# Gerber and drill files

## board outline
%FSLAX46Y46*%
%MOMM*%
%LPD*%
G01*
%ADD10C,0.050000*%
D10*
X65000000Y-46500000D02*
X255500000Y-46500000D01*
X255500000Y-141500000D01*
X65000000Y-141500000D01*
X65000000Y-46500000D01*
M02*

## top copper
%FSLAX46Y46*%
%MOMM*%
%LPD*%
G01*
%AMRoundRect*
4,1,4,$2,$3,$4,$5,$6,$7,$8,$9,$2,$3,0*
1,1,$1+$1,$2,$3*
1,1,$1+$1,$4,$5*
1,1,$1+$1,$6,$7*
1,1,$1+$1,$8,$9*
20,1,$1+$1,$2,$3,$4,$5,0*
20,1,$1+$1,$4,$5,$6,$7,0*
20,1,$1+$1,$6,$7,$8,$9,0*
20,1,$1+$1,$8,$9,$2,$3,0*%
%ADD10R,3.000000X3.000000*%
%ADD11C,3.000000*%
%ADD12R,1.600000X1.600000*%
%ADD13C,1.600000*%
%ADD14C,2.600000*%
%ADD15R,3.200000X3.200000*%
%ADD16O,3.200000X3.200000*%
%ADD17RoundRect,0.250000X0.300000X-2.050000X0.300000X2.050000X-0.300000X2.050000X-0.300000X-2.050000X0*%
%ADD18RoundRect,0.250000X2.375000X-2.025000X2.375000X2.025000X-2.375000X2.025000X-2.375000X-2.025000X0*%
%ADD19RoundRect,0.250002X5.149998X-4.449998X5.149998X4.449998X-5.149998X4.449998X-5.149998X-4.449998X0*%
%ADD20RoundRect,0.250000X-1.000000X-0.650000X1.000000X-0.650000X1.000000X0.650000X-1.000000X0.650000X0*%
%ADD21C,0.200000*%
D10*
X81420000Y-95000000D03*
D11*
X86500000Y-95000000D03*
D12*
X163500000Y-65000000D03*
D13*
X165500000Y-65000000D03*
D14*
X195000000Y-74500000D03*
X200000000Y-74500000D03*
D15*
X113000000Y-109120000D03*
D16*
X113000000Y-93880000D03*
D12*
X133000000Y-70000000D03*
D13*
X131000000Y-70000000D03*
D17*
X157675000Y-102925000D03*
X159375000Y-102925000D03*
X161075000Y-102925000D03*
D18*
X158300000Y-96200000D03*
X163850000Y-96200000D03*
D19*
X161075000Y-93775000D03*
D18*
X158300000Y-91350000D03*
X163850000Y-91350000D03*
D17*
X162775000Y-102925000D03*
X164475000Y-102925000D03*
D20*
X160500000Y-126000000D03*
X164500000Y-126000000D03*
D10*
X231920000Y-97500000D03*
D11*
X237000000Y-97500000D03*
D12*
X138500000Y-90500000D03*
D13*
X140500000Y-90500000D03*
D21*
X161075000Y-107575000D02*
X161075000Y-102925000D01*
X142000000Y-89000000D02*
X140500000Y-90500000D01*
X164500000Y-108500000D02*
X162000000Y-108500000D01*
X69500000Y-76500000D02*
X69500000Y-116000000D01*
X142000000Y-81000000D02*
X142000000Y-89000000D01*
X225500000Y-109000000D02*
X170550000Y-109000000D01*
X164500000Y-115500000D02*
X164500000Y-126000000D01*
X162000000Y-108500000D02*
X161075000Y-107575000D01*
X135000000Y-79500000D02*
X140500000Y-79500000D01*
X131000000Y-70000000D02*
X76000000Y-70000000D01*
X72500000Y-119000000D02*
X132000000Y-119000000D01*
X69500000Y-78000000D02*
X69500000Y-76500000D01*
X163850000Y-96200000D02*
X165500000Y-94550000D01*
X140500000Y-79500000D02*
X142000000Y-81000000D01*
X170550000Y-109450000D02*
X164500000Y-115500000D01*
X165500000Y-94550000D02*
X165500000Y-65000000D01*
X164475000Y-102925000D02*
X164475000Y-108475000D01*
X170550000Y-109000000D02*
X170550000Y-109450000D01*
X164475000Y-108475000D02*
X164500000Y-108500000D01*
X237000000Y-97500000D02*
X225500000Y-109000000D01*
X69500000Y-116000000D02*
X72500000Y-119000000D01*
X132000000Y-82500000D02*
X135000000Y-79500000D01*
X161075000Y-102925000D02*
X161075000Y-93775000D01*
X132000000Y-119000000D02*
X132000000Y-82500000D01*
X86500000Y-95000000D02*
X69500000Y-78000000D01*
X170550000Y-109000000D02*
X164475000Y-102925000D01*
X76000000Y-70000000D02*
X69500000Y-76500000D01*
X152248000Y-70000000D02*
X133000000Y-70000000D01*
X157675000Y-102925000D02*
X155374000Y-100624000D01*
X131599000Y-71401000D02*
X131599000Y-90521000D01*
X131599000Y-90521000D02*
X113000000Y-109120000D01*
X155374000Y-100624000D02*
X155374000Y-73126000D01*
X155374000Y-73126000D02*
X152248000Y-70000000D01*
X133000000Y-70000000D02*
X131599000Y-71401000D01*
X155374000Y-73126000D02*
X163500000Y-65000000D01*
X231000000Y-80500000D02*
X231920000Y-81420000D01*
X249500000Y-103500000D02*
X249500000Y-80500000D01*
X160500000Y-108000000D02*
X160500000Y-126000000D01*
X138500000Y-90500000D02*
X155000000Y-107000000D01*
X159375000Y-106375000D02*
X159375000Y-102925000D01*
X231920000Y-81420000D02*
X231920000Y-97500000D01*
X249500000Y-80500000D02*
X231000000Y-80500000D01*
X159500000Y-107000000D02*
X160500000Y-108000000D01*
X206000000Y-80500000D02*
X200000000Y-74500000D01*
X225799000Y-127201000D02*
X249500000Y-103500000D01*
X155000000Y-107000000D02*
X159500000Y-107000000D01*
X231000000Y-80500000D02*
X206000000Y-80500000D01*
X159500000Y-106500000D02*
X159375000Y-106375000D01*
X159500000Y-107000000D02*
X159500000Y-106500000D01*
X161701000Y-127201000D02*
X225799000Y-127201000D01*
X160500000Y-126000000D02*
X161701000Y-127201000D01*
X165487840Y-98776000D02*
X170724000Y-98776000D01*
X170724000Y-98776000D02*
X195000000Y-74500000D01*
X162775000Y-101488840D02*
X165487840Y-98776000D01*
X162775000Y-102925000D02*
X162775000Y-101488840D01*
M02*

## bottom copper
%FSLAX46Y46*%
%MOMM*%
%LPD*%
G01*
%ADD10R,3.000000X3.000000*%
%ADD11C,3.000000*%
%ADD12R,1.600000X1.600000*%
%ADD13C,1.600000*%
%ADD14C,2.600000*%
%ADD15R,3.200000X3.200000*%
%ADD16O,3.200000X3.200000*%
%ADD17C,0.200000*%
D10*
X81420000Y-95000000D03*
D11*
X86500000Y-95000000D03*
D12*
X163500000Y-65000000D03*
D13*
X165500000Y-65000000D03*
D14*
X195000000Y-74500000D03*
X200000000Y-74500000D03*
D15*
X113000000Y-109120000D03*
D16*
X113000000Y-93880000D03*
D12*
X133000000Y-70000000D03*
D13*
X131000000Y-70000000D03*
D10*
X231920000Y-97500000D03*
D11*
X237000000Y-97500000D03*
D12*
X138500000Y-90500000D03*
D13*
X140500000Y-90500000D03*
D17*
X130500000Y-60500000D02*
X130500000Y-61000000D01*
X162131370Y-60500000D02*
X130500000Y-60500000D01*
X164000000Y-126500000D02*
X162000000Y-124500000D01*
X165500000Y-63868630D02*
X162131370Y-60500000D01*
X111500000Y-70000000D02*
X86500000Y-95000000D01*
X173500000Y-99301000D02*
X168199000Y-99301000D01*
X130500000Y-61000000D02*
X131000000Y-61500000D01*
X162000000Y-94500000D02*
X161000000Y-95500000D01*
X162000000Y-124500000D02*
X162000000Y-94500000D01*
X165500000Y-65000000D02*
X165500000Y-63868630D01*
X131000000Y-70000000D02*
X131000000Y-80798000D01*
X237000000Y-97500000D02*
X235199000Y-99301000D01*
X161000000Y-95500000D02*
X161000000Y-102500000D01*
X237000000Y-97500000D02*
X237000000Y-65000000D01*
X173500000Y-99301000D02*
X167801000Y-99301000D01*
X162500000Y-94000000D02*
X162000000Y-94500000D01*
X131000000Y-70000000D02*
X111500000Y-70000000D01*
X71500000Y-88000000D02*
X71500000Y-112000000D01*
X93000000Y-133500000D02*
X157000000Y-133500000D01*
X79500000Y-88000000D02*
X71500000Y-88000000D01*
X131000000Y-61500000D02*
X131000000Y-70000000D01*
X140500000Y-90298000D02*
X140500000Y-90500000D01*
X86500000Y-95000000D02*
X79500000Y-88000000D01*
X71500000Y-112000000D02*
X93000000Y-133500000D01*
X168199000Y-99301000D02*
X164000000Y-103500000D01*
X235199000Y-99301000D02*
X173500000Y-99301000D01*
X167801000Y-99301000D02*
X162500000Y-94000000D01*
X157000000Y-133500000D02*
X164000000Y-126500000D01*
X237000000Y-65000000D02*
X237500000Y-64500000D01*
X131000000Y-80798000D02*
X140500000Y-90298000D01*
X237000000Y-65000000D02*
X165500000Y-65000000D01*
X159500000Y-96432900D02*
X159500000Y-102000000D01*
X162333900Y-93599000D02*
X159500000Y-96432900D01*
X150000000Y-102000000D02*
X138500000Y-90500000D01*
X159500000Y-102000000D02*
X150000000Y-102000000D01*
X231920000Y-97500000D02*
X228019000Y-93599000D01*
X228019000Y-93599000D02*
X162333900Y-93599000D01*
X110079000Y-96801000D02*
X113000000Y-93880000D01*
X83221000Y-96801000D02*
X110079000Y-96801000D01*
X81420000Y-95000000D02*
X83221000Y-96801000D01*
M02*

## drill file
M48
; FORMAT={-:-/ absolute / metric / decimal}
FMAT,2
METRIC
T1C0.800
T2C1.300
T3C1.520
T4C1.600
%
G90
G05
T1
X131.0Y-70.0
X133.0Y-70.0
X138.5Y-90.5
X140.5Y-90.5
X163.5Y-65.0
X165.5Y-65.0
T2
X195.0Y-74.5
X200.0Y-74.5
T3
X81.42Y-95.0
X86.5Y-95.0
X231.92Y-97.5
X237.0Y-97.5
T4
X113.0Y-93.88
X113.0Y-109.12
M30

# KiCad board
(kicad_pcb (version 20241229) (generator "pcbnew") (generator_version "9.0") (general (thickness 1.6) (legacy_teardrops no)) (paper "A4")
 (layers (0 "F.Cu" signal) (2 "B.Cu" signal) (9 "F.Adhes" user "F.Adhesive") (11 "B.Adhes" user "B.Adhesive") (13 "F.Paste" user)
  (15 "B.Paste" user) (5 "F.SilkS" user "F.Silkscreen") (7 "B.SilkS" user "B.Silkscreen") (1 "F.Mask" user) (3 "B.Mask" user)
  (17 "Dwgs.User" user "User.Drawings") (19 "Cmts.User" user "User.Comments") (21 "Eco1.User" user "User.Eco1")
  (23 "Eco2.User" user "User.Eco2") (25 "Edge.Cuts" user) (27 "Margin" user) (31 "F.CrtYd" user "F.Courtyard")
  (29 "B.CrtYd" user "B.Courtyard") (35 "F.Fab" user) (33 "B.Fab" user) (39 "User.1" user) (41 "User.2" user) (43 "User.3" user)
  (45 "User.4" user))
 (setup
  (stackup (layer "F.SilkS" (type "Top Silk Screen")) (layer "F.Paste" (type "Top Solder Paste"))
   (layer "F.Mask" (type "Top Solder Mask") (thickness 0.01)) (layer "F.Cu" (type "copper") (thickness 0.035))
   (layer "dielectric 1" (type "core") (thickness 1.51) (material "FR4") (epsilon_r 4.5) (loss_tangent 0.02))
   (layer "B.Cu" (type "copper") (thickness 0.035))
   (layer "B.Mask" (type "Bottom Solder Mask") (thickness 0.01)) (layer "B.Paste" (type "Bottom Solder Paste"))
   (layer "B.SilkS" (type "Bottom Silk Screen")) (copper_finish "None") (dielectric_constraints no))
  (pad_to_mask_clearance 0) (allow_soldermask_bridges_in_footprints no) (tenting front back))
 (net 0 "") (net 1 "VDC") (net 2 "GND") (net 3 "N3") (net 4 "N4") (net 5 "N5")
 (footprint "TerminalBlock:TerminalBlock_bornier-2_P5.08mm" (layer "F.Cu") (at 81.42 95)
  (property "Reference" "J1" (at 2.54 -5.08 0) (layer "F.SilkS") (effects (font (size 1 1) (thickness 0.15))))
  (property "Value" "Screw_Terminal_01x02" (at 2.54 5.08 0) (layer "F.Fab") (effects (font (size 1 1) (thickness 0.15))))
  (pad "1" thru_hole rect (at 0 0) (size 3 3) (drill 1.52) (layers "*.Cu" "*.Mask") (remove_unused_layers no) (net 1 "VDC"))
  (pad "2" thru_hole circle (at 5.08 0) (size 3 3) (drill 1.52) (layers "*.Cu" "*.Mask") (remove_unused_layers no) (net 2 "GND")))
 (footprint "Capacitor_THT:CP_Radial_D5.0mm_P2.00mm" (layer "F.Cu") (at 163.5 65)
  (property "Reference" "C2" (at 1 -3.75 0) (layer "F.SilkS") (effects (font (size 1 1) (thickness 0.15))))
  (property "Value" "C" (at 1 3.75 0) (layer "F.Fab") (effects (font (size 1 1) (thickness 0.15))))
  (pad "1" thru_hole rect (at 0 0) (size 1.6 1.6) (drill 0.8) (layers "*.Cu" "*.Mask") (remove_unused_layers no) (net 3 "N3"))
  (pad "2" thru_hole circle (at 2 0) (size 1.6 1.6) (drill 0.8) (layers "*.Cu" "*.Mask") (remove_unused_layers no) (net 2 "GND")))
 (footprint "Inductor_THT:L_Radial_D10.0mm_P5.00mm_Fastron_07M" (layer "F.Cu") (at 195 74.5)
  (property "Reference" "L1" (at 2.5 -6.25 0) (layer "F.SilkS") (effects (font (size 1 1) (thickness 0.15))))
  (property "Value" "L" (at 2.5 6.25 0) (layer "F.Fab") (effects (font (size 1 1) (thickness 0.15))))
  (pad "1" thru_hole circle (at 0 0) (size 2.6 2.6) (drill 1.3) (layers "*.Cu" "*.Mask") (remove_unused_layers no) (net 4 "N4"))
  (pad "2" thru_hole circle (at 5 0) (size 2.6 2.6) (drill 1.3) (layers "*.Cu" "*.Mask") (remove_unused_layers no) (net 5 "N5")))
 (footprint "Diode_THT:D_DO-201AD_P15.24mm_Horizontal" (layer "F.Cu") (at 113 109.12 90)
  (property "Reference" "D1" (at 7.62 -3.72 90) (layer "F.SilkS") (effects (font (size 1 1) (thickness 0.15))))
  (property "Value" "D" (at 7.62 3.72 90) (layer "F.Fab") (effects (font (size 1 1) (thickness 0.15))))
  (pad "1" thru_hole rect (at 0 0 90) (size 3.2 3.2) (drill 1.6) (layers "*.Cu" "*.Mask") (remove_unused_layers no) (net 3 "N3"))
  (pad "2" thru_hole oval (at 15.24 0 90) (size 3.2 3.2) (drill 1.6) (layers "*.Cu" "*.Mask") (remove_unused_layers no) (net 1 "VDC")))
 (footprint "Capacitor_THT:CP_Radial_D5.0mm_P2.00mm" (layer "F.Cu") (at 133 70 180)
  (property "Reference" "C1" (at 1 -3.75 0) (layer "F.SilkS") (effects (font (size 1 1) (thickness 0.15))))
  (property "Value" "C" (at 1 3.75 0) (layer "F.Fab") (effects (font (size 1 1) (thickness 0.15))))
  (pad "1" thru_hole rect (at 0 0 180) (size 1.6 1.6) (drill 0.8) (layers "*.Cu" "*.Mask") (remove_unused_layers no) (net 3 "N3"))
  (pad "2" thru_hole circle (at 2 0 180) (size 1.6 1.6) (drill 0.8) (layers "*.Cu" "*.Mask") (remove_unused_layers no) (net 2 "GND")))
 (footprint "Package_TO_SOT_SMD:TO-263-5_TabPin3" (layer "F.Cu") (at 161.075 95.275 90)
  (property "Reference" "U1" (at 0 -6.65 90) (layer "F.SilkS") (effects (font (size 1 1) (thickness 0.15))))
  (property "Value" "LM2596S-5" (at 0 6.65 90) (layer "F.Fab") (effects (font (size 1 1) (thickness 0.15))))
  (pad "1" smd roundrect (at -7.65 -3.4 90) (size 4.6 1.1) (layers "F.Cu" "F.Mask" "F.Paste") (roundrect_rratio 0.227273) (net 3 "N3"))
  (pad "2" smd roundrect (at -7.65 -1.7 90) (size 4.6 1.1) (layers "F.Cu" "F.Mask" "F.Paste") (roundrect_rratio 0.227273) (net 5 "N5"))
  (pad "3" smd roundrect (at -7.65 0 90) (size 4.6 1.1) (layers "F.Cu" "F.Mask" "F.Paste") (roundrect_rratio 0.227273) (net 2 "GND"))
  (pad "3" smd roundrect (at -0.925 -2.775 90) (size 4.55 5.25) (layers "F.Cu" "F.Paste") (roundrect_rratio 0.054945) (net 2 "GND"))
  (pad "3" smd roundrect (at -0.925 2.775 90) (size 4.55 5.25) (layers "F.Cu" "F.Paste") (roundrect_rratio 0.054945) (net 2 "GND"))
  (pad "3" smd roundrect (at 1.5 0 90) (size 9.4 10.8) (layers "F.Cu" "F.Mask") (roundrect_rratio 0.026596) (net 2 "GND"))
  (pad "3" smd roundrect (at 3.925 -2.775 90) (size 4.55 5.25) (layers "F.Cu" "F.Paste") (roundrect_rratio 0.054945) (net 2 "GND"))
  (pad "3" smd roundrect (at 3.925 2.775 90) (size 4.55 5.25) (layers "F.Cu" "F.Paste") (roundrect_rratio 0.054945) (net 2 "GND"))
  (pad "4" smd roundrect (at -7.65 1.7 90) (size 4.6 1.1) (layers "F.Cu" "F.Mask" "F.Paste") (roundrect_rratio 0.227273) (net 4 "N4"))
  (pad "5" smd roundrect (at -7.65 3.4 90) (size 4.6 1.1) (layers "F.Cu" "F.Mask" "F.Paste") (roundrect_rratio 0.227273) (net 2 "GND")))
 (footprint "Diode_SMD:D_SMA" (layer "F.Cu") (at 162.5 126)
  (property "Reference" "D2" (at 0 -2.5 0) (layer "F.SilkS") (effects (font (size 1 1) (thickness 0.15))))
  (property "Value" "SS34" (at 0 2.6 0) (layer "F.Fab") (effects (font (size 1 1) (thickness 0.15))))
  (pad "1" smd roundrect (at -2 0) (size 2.5 1.8) (layers "F.Cu" "F.Mask" "F.Paste") (roundrect_rratio 0.1388888889) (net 5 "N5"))
  (pad "2" smd roundrect (at 2 0) (size 2.5 1.8) (layers "F.Cu" "F.Mask" "F.Paste") (roundrect_rratio 0.1388888889) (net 2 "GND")))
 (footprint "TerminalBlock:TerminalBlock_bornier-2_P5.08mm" (layer "F.Cu") (at 231.92 97.5)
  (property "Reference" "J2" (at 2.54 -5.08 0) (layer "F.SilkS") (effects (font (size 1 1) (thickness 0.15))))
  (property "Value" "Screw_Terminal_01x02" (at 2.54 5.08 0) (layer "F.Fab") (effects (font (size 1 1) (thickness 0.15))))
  (pad "1" thru_hole rect (at 0 0) (size 3 3) (drill 1.52) (layers "*.Cu" "*.Mask") (remove_unused_layers no) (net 5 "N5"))
  (pad "2" thru_hole circle (at 5.08 0) (size 3 3) (drill 1.52) (layers "*.Cu" "*.Mask") (remove_unused_layers no) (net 2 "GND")))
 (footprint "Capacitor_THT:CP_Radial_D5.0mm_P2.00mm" (layer "F.Cu") (at 138.5 90.5)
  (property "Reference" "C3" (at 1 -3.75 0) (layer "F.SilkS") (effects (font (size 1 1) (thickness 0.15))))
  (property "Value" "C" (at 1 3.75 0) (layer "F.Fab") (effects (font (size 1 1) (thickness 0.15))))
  (pad "1" thru_hole rect (at 0 0) (size 1.6 1.6) (drill 0.8) (layers "*.Cu" "*.Mask") (remove_unused_layers no) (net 5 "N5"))
  (pad "2" thru_hole circle (at 2 0) (size 1.6 1.6) (drill 0.8) (layers "*.Cu" "*.Mask") (remove_unused_layers no) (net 2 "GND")))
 (gr_rect (start 65 46.5) (end 255.5 141.5) (stroke (width 0.05) (type default)) (fill no) (layer "Edge.Cuts"))
 (segment (start 161.075 107.575) (end 161.075 102.925) (width 0.2) (layer "F.Cu") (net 2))
 (segment (start 142 89) (end 140.5 90.5) (width 0.2) (layer "F.Cu") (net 2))
 (segment (start 164.5 108.5) (end 162 108.5) (width 0.2) (layer "F.Cu") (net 2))
 (segment (start 69.5 76.5) (end 69.5 116) (width 0.2) (layer "F.Cu") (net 2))
 (segment (start 142 81) (end 142 89) (width 0.2) (layer "F.Cu") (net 2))
 (segment (start 225.5 109) (end 170.55 109) (width 0.2) (layer "F.Cu") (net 2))
 (segment (start 164.5 115.5) (end 164.5 126) (width 0.2) (layer "F.Cu") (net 2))
 (segment (start 162 108.5) (end 161.075 107.575) (width 0.2) (layer "F.Cu") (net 2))
 (segment (start 135 79.5) (end 140.5 79.5) (width 0.2) (layer "F.Cu") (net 2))
 (segment (start 131 70) (end 76 70) (width 0.2) (layer "F.Cu") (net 2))
 (segment (start 72.5 119) (end 132 119) (width 0.2) (layer "F.Cu") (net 2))
 (segment (start 69.5 78) (end 69.5 76.5) (width 0.2) (layer "F.Cu") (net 2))
 (segment (start 163.85 96.2) (end 165.5 94.55) (width 0.2) (layer "F.Cu") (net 2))
 (segment (start 140.5 79.5) (end 142 81) (width 0.2) (layer "F.Cu") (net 2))
 (segment (start 170.55 109.45) (end 164.5 115.5) (width 0.2) (layer "F.Cu") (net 2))
 (segment (start 165.5 94.55) (end 165.5 65) (width 0.2) (layer "F.Cu") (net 2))
 (segment (start 164.475 102.925) (end 164.475 108.475) (width 0.2) (layer "F.Cu") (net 2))
 (segment (start 170.55 109) (end 170.55 109.45) (width 0.2) (layer "F.Cu") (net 2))
 (segment (start 164.475 108.475) (end 164.5 108.5) (width 0.2) (layer "F.Cu") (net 2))
 (segment (start 237 97.5) (end 225.5 109) (width 0.2) (layer "F.Cu") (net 2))
 (segment (start 69.5 116) (end 72.5 119) (width 0.2) (layer "F.Cu") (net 2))
 (segment (start 132 82.5) (end 135 79.5) (width 0.2) (layer "F.Cu") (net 2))
 (segment (start 161.075 102.925) (end 161.075 93.775) (width 0.2) (layer "F.Cu") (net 2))
 (segment (start 132 119) (end 132 82.5) (width 0.2) (layer "F.Cu") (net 2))
 (segment (start 86.5 95) (end 69.5 78) (width 0.2) (layer "F.Cu") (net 2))
 (segment (start 170.55 109) (end 164.475 102.925) (width 0.2) (layer "F.Cu") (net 2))
 (segment (start 76 70) (end 69.5 76.5) (width 0.2) (layer "F.Cu") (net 2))
 (segment (start 130.5 60.5) (end 130.5 61) (width 0.2) (layer "B.Cu") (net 2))
 (segment (start 162.13137 60.5) (end 130.5 60.5) (width 0.2) (layer "B.Cu") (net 2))
 (segment (start 164 126.5) (end 162 124.5) (width 0.2) (layer "B.Cu") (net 2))
 (segment (start 165.5 63.86863) (end 162.13137 60.5) (width 0.2) (layer "B.Cu") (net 2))
 (segment (start 111.5 70) (end 86.5 95) (width 0.2) (layer "B.Cu") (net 2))
 (segment (start 173.5 99.301) (end 168.199 99.301) (width 0.2) (layer "B.Cu") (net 2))
 (segment (start 130.5 61) (end 131 61.5) (width 0.2) (layer "B.Cu") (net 2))
 (segment (start 162 94.5) (end 161 95.5) (width 0.2) (layer "B.Cu") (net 2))
 (segment (start 162 124.5) (end 162 94.5) (width 0.2) (layer "B.Cu") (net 2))
 (segment (start 165.5 65) (end 165.5 63.86863) (width 0.2) (layer "B.Cu") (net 2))
 (segment (start 131 70) (end 131 80.798) (width 0.2) (layer "B.Cu") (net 2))
 (segment (start 237 97.5) (end 235.199 99.301) (width 0.2) (layer "B.Cu") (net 2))
 (segment (start 161 95.5) (end 161 102.5) (width 0.2) (layer "B.Cu") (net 2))
 (segment (start 237 97.5) (end 237 65) (width 0.2) (layer "B.Cu") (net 2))
 (segment (start 173.5 99.301) (end 167.801 99.301) (width 0.2) (layer "B.Cu") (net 2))
 (segment (start 162.5 94) (end 162 94.5) (width 0.2) (layer "B.Cu") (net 2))
 (segment (start 131 70) (end 111.5 70) (width 0.2) (layer "B.Cu") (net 2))
 (segment (start 71.5 88) (end 71.5 112) (width 0.2) (layer "B.Cu") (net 2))
 (segment (start 93 133.5) (end 157 133.5) (width 0.2) (layer "B.Cu") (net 2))
 (segment (start 79.5 88) (end 71.5 88) (width 0.2) (layer "B.Cu") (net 2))
 (segment (start 131 61.5) (end 131 70) (width 0.2) (layer "B.Cu") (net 2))
 (segment (start 140.5 90.298) (end 140.5 90.5) (width 0.2) (layer "B.Cu") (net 2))
 (segment (start 86.5 95) (end 79.5 88) (width 0.2) (layer "B.Cu") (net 2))
 (segment (start 71.5 112) (end 93 133.5) (width 0.2) (layer "B.Cu") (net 2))
 (segment (start 168.199 99.301) (end 164 103.5) (width 0.2) (layer "B.Cu") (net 2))
 (segment (start 235.199 99.301) (end 173.5 99.301) (width 0.2) (layer "B.Cu") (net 2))
 (segment (start 167.801 99.301) (end 162.5 94) (width 0.2) (layer "B.Cu") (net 2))
 (segment (start 157 133.5) (end 164 126.5) (width 0.2) (layer "B.Cu") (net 2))
 (segment (start 237 65) (end 237.5 64.5) (width 0.2) (layer "B.Cu") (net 2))
 (segment (start 131 80.798) (end 140.5 90.298) (width 0.2) (layer "B.Cu") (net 2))
 (segment (start 237 65) (end 165.5 65) (width 0.2) (layer "B.Cu") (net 2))
 (segment (start 152.248 70) (end 133 70) (width 0.2) (layer "F.Cu") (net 3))
 (segment (start 157.675 102.925) (end 155.374 100.624) (width 0.2) (layer "F.Cu") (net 3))
 (segment (start 131.599 71.401) (end 131.599 90.521) (width 0.2) (layer "F.Cu") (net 3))
 (segment (start 131.599 90.521) (end 113 109.12) (width 0.2) (layer "F.Cu") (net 3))
 (segment (start 155.374 100.624) (end 155.374 73.126) (width 0.2) (layer "F.Cu") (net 3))
 (segment (start 155.374 73.126) (end 152.248 70) (width 0.2) (layer "F.Cu") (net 3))
 (segment (start 133 70) (end 131.599 71.401) (width 0.2) (layer "F.Cu") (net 3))
 (segment (start 155.374 73.126) (end 163.5 65) (width 0.2) (layer "F.Cu") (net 3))
 (segment (start 231 80.5) (end 231.92 81.42) (width 0.2) (layer "F.Cu") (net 5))
 (segment (start 249.5 103.5) (end 249.5 80.5) (width 0.2) (layer "F.Cu") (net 5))
 (segment (start 160.5 108) (end 160.5 126) (width 0.2) (layer "F.Cu") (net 5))
 (segment (start 138.5 90.5) (end 155 107) (width 0.2) (layer "F.Cu") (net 5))
 (segment (start 159.375 106.375) (end 159.375 102.925) (width 0.2) (layer "F.Cu") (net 5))
 (segment (start 231.92 81.42) (end 231.92 97.5) (width 0.2) (layer "F.Cu") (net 5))
 (segment (start 249.5 80.5) (end 231 80.5) (width 0.2) (layer "F.Cu") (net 5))
 (segment (start 159.5 107) (end 160.5 108) (width 0.2) (layer "F.Cu") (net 5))
 (segment (start 206 80.5) (end 200 74.5) (width 0.2) (layer "F.Cu") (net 5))
 (segment (start 225.799 127.201) (end 249.5 103.5) (width 0.2) (layer "F.Cu") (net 5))
 (segment (start 155 107) (end 159.5 107) (width 0.2) (layer "F.Cu") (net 5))
 (segment (start 231 80.5) (end 206 80.5) (width 0.2) (layer "F.Cu") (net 5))
 (segment (start 159.5 106.5) (end 159.375 106.375) (width 0.2) (layer "F.Cu") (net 5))
 (segment (start 159.5 107) (end 159.5 106.5) (width 0.2) (layer "F.Cu") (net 5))
 (segment (start 161.701 127.201) (end 225.799 127.201) (width 0.2) (layer "F.Cu") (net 5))
 (segment (start 160.5 126) (end 161.701 127.201) (width 0.2) (layer "F.Cu") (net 5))
 (segment (start 159.5 96.4329) (end 159.5 102) (width 0.2) (layer "B.Cu") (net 5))
 (segment (start 162.3339 93.599) (end 159.5 96.4329) (width 0.2) (layer "B.Cu") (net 5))
 (segment (start 150 102) (end 138.5 90.5) (width 0.2) (layer "B.Cu") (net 5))
 (segment (start 159.5 102) (end 150 102) (width 0.2) (layer "B.Cu") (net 5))
 (segment (start 231.92 97.5) (end 228.019 93.599) (width 0.2) (layer "B.Cu") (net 5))
 (segment (start 228.019 93.599) (end 162.3339 93.599) (width 0.2) (layer "B.Cu") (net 5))
 (segment (start 110.079 96.801) (end 113 93.88) (width 0.2) (layer "B.Cu") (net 1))
 (segment (start 83.221 96.801) (end 110.079 96.801) (width 0.2) (layer "B.Cu") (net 1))
 (segment (start 81.42 95) (end 83.221 96.801) (width 0.2) (layer "B.Cu") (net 1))
 (segment (start 165.48784 98.776) (end 170.724 98.776) (width 0.2) (layer "F.Cu") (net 4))
 (segment (start 170.724 98.776) (end 195 74.5) (width 0.2) (layer "F.Cu") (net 4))
 (segment (start 162.775 101.48884) (end 165.48784 98.776) (width 0.2) (layer "F.Cu") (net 4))
 (segment (start 162.775 102.925) (end 162.775 101.48884) (width 0.2) (layer "F.Cu") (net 4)))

